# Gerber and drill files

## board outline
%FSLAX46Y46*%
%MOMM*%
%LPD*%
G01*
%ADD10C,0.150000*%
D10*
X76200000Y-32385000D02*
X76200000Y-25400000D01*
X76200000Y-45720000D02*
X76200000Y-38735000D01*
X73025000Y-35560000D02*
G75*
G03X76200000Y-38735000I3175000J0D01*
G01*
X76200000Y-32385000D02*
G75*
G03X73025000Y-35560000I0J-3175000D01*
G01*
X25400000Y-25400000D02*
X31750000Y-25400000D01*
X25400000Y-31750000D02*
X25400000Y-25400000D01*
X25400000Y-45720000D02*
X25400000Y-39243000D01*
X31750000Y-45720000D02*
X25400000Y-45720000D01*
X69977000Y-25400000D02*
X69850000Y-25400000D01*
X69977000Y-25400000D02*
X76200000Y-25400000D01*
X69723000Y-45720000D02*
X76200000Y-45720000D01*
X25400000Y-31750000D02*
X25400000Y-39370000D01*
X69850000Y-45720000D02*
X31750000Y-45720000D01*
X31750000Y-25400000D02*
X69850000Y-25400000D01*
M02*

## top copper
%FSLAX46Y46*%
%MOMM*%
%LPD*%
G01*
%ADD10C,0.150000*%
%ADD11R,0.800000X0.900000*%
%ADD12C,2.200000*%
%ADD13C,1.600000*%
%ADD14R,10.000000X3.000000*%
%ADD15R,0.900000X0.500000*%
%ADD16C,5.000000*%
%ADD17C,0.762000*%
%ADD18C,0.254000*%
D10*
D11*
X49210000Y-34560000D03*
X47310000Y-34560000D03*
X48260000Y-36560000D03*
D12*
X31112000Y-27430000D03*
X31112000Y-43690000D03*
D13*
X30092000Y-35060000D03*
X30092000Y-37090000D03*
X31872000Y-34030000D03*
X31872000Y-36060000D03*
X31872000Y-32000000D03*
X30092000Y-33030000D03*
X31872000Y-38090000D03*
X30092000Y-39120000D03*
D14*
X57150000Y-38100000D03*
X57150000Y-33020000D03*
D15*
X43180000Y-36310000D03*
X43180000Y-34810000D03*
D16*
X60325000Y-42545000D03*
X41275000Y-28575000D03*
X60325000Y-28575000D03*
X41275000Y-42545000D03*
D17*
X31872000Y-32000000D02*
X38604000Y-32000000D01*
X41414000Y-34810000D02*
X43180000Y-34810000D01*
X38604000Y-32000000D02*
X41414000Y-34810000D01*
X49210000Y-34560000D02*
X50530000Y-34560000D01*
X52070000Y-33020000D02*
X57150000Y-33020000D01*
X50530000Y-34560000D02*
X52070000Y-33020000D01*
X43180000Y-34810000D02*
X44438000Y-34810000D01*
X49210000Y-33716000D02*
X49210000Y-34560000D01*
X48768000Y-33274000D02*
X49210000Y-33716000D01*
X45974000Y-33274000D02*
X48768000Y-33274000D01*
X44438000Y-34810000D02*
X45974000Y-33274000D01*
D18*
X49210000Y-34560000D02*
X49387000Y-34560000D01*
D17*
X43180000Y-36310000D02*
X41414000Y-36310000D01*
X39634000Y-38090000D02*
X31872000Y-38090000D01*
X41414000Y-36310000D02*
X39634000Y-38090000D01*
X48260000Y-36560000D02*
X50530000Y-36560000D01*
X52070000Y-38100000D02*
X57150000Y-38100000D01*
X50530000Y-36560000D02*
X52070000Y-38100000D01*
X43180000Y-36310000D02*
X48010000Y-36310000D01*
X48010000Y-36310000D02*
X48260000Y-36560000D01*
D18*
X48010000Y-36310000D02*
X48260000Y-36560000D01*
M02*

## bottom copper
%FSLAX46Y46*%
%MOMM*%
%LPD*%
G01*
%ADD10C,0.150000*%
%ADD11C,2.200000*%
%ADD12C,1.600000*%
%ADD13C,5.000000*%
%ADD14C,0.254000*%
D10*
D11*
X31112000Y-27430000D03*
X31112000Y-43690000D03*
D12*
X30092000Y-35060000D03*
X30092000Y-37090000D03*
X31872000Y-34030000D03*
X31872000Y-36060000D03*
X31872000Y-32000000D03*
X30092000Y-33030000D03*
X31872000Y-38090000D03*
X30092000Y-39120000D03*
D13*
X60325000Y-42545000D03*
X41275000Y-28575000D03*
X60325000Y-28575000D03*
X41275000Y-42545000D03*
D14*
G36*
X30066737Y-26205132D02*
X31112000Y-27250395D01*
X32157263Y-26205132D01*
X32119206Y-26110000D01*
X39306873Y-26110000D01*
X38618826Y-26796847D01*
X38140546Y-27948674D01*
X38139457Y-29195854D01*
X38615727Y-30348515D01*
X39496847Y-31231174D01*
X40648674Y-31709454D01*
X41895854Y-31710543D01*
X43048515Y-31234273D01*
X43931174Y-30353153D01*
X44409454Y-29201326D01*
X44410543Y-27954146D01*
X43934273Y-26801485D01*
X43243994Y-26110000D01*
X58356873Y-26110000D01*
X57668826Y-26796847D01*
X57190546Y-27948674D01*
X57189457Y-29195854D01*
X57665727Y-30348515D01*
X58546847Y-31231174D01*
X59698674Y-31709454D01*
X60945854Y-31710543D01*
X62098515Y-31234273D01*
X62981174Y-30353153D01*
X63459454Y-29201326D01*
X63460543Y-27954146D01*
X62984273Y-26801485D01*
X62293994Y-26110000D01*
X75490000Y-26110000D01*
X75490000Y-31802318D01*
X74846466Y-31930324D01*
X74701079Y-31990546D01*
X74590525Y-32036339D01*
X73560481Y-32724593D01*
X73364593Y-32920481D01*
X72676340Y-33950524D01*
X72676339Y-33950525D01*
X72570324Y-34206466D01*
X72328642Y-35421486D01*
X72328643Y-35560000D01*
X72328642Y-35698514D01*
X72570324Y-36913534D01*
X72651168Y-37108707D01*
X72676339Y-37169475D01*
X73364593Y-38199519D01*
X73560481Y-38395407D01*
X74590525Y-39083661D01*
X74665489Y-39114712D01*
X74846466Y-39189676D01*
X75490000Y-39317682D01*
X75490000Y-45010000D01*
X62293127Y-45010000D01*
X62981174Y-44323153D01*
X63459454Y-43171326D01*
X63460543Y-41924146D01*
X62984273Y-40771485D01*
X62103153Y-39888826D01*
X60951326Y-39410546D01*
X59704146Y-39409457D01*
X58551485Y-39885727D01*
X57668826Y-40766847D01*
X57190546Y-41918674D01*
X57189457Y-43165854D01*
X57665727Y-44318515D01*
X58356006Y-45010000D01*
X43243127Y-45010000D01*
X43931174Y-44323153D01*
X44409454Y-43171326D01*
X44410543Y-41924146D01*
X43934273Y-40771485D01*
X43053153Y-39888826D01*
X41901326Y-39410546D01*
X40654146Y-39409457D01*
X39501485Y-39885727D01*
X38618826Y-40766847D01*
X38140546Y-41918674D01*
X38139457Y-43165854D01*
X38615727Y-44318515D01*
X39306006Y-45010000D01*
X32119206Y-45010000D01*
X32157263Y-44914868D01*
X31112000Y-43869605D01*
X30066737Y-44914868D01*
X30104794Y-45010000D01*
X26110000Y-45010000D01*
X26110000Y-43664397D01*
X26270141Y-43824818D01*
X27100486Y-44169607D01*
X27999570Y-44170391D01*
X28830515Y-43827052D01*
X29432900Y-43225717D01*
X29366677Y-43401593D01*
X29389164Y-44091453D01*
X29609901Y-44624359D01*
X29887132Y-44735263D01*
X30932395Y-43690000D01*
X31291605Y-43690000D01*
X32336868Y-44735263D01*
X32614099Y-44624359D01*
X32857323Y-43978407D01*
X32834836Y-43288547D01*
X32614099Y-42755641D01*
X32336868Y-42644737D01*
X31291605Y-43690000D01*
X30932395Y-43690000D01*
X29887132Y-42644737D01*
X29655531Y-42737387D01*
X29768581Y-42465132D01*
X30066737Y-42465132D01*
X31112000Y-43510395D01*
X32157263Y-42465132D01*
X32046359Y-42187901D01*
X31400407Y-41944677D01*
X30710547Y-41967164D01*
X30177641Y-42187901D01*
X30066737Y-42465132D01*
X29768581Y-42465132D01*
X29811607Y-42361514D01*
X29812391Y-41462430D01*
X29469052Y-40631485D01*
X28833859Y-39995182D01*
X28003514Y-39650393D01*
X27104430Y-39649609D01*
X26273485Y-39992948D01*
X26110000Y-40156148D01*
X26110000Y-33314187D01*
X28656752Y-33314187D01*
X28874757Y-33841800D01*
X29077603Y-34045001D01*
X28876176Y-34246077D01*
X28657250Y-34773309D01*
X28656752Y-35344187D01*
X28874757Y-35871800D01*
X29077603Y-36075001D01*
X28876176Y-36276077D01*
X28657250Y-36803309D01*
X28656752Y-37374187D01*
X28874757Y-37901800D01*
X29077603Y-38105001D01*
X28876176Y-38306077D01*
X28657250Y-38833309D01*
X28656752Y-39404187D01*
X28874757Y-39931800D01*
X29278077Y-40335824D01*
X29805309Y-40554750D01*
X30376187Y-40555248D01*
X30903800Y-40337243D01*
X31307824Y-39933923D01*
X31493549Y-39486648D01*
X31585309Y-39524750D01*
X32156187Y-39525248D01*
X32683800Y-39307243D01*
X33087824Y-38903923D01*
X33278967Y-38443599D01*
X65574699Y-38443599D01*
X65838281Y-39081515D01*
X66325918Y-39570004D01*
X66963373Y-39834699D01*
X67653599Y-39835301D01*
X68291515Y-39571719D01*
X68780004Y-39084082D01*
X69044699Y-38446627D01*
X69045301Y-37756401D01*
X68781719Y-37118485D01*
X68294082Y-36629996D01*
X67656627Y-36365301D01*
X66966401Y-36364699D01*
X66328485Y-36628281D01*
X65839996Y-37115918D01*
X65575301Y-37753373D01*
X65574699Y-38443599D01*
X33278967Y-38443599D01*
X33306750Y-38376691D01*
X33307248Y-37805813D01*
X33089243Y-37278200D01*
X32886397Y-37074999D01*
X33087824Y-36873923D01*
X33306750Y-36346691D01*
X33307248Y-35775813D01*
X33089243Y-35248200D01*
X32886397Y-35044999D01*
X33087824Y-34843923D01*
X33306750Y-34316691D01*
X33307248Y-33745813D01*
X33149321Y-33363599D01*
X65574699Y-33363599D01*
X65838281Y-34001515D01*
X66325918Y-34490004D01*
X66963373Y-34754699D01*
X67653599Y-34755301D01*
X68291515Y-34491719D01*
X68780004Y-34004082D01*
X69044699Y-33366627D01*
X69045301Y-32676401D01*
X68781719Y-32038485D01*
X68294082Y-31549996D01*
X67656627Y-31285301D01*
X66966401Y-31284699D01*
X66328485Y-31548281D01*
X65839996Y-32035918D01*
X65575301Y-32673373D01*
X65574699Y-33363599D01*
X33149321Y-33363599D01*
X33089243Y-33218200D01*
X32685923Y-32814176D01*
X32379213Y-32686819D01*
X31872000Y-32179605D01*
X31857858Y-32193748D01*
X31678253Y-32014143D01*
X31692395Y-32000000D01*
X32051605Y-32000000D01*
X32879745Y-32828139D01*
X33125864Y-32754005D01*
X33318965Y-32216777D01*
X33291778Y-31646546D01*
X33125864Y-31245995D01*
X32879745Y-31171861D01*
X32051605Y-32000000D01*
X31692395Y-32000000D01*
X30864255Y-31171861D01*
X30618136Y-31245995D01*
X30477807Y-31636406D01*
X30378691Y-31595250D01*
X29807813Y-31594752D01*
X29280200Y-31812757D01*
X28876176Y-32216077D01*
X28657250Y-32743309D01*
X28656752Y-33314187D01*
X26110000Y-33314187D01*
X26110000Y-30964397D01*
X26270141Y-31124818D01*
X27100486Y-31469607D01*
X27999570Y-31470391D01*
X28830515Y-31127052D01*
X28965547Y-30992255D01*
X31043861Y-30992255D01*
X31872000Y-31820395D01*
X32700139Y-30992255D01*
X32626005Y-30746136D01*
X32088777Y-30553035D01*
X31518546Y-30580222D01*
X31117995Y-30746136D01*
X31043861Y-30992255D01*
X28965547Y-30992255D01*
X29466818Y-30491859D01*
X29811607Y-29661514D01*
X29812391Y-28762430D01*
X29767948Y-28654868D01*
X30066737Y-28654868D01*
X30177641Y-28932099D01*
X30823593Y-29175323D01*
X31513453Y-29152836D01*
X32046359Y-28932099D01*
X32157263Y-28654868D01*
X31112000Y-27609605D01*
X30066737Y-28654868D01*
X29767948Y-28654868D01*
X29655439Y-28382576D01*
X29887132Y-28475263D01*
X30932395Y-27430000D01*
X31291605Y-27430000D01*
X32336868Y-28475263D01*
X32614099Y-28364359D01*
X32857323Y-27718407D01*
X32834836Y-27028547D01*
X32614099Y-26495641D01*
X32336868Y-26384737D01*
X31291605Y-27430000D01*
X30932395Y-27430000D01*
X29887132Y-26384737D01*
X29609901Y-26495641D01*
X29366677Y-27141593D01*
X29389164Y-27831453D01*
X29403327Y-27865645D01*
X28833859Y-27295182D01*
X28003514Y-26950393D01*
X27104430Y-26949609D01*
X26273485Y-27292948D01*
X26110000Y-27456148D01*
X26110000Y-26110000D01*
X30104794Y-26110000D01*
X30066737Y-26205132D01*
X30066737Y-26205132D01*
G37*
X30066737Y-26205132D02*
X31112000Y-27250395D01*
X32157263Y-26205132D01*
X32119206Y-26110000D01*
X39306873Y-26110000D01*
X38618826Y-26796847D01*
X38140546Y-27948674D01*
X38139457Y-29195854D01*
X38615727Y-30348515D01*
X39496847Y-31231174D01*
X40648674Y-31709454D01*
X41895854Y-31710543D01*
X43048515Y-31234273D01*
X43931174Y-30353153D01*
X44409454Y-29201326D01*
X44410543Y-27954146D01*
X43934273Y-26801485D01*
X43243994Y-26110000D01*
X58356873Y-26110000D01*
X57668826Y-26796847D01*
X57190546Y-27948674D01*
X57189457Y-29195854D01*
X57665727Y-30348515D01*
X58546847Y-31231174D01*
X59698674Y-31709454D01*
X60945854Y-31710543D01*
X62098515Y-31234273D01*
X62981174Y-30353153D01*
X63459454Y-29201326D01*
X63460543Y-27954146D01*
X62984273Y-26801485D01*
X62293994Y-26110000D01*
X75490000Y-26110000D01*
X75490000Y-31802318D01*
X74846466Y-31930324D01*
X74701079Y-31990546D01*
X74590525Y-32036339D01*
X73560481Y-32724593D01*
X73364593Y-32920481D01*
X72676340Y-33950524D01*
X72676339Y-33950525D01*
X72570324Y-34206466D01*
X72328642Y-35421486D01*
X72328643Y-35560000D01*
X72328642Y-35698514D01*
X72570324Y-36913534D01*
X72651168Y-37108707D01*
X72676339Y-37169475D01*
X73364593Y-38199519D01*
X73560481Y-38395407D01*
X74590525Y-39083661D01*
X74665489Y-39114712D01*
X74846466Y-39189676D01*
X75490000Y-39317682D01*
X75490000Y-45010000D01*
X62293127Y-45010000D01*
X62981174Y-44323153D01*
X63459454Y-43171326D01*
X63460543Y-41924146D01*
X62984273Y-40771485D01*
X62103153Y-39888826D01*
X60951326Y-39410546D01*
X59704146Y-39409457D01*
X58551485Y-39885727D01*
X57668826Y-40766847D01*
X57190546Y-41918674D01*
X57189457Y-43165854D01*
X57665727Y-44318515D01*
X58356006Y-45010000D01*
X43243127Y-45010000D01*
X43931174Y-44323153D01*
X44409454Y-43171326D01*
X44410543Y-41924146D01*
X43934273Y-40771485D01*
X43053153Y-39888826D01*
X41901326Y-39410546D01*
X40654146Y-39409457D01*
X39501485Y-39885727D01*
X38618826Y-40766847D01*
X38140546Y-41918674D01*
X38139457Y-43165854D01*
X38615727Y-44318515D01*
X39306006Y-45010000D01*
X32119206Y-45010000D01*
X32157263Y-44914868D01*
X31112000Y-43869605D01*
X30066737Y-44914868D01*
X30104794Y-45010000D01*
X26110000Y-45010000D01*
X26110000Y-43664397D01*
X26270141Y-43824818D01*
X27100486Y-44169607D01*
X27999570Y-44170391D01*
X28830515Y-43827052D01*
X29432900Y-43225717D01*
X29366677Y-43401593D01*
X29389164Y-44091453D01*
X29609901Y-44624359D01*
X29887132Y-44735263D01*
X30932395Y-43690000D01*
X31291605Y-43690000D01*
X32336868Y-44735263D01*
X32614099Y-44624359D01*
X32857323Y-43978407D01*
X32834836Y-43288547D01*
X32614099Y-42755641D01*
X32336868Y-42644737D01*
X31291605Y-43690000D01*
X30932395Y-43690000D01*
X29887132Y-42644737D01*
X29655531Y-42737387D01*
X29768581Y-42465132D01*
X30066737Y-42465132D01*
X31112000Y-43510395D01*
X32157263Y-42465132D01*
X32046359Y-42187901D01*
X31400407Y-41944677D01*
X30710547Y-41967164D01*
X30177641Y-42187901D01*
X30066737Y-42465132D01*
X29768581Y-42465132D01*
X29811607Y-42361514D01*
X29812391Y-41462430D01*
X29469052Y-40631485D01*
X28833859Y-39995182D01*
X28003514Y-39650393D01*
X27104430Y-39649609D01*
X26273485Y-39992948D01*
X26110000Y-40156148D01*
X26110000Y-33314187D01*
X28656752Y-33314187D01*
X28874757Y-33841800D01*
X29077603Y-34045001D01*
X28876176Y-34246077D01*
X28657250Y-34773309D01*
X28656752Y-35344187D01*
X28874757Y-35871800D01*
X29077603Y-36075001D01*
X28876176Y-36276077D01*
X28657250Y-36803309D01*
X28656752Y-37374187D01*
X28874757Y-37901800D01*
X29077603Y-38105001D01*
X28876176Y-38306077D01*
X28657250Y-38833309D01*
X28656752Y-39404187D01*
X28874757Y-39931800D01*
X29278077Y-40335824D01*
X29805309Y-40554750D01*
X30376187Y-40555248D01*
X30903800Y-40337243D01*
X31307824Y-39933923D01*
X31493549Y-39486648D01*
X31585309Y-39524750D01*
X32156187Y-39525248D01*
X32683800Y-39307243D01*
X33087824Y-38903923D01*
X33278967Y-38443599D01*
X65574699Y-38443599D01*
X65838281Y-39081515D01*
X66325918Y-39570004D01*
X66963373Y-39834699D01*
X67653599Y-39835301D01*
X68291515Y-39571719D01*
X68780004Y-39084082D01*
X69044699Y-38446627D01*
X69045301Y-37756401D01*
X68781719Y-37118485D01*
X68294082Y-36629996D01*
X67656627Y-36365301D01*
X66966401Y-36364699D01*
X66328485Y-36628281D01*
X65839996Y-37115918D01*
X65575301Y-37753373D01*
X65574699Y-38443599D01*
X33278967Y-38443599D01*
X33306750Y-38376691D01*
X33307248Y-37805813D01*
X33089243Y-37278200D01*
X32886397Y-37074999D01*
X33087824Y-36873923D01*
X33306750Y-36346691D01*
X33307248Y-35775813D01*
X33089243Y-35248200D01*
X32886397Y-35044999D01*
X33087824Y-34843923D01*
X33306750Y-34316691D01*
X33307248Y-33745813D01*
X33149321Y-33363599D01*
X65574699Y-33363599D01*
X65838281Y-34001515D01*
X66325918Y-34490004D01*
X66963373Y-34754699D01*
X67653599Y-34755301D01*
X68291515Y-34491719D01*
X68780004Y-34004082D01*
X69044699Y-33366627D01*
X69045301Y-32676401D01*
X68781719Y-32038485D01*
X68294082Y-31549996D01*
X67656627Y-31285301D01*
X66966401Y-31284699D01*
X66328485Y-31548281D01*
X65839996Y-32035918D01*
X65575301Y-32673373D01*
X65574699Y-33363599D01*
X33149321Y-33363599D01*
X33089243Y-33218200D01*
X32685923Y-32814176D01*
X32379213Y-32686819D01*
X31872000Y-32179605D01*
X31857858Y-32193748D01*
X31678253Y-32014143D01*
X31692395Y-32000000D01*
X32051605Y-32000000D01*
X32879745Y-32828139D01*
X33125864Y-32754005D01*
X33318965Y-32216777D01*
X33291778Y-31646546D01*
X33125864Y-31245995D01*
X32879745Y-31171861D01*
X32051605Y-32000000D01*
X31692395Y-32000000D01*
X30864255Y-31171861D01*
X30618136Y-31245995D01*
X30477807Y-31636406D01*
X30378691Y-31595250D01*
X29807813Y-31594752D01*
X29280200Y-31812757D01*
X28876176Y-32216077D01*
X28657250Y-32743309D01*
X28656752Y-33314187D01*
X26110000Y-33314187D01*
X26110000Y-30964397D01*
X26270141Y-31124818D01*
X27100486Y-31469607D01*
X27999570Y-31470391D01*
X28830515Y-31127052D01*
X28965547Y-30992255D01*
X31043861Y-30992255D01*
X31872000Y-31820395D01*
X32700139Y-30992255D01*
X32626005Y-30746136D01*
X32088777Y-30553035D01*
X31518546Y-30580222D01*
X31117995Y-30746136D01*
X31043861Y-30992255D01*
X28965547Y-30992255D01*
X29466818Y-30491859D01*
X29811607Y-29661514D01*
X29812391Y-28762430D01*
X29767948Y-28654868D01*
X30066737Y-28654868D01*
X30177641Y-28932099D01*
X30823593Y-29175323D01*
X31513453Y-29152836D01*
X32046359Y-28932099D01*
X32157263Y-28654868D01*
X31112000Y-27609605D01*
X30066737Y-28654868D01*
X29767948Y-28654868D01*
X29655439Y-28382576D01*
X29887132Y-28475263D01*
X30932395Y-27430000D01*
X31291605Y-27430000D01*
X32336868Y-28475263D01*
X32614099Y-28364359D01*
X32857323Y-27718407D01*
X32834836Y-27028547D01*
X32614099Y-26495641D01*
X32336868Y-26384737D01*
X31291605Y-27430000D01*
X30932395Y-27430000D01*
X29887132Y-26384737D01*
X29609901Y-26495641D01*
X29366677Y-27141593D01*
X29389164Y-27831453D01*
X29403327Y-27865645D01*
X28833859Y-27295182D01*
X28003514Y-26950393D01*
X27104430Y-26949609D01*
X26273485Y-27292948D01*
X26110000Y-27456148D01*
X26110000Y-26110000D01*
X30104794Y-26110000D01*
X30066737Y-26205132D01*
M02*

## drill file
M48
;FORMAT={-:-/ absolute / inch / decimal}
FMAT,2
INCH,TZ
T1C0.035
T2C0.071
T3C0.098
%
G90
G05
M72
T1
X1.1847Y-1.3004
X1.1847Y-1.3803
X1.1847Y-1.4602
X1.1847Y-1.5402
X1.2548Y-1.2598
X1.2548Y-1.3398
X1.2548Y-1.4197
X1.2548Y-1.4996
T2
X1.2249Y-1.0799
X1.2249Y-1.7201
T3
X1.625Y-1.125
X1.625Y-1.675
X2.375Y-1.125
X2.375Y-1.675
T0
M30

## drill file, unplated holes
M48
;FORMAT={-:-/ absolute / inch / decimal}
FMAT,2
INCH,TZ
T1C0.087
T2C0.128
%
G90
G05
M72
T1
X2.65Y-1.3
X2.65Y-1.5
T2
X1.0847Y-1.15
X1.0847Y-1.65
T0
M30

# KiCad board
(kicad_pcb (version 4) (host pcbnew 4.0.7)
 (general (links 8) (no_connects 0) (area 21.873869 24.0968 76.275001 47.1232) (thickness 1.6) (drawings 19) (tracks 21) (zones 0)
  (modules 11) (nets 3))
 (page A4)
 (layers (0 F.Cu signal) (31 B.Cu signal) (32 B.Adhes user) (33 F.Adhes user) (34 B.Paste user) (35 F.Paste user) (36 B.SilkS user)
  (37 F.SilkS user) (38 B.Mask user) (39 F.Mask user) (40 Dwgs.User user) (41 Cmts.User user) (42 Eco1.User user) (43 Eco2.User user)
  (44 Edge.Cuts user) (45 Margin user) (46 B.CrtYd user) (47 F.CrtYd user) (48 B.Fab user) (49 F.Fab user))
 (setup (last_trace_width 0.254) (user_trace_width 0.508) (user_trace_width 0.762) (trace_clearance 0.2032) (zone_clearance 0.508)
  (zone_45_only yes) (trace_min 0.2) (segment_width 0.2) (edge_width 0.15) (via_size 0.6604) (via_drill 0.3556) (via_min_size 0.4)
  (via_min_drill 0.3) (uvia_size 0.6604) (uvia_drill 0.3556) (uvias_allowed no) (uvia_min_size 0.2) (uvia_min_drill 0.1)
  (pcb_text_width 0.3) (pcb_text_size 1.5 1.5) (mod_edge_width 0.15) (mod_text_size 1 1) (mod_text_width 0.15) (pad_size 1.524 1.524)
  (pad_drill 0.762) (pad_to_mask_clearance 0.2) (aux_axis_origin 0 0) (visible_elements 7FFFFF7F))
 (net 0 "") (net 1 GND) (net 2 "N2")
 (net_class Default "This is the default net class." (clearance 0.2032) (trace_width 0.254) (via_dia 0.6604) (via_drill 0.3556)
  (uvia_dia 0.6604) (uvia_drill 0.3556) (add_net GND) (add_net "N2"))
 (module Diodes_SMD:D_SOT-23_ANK (layer F.Cu) (at 48.26 35.56 270)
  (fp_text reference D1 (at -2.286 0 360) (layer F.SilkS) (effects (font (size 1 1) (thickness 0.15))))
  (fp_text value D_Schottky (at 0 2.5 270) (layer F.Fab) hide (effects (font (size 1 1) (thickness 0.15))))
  (pad 2 smd rect (at -1 -0.95 270) (size 0.9 0.8) (layers F.Cu F.Paste F.Mask) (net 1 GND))
  (pad "" smd rect (at -1 0.95 270) (size 0.9 0.8) (layers F.Cu F.Paste F.Mask))
  (pad 1 smd rect (at 1 0 270) (size 0.9 0.8) (layers F.Cu F.Paste F.Mask) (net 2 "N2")))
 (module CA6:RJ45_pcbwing (layer F.Cu) (at 29.972 35.56 270)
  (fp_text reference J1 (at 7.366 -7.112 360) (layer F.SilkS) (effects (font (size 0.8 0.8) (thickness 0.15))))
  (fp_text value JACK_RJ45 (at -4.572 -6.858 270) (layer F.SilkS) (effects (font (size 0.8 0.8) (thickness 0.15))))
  (pad 8 thru_hole circle (at -8.13 -1.14 270) (size 2.2 2.2) (drill 1.8) (layers *.Cu *.Mask F.SilkS) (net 1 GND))
  (pad 8 thru_hole circle (at 8.13 -1.14 270) (size 2.2 2.2) (drill 1.8) (layers *.Cu *.Mask F.SilkS) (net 1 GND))
  (pad "" np_thru_hole circle (at -6.35 2.42 270) (size 3.25 3.25) (drill 3.25) (layers *.Cu *.Mask F.SilkS))
  (pad "" np_thru_hole circle (at 6.35 2.42 270) (size 3.25 3.25) (drill 3.25) (layers *.Cu *.Mask F.SilkS))
  (pad 5 thru_hole circle (at -0.5 -0.12 270) (size 1.6 1.6) (drill 0.89) (layers *.Cu *.Mask F.SilkS))
  (pad 3 thru_hole circle (at 1.53 -0.12 270) (size 1.6 1.6) (drill 0.89) (layers *.Cu *.Mask F.SilkS))
  (pad 6 thru_hole circle (at -1.53 -1.9 270) (size 1.6 1.6) (drill 0.89) (layers *.Cu *.Mask F.SilkS))
  (pad 4 thru_hole circle (at 0.5 -1.9 270) (size 1.6 1.6) (drill 0.89) (layers *.Cu *.Mask F.SilkS))
  (pad 8 thru_hole circle (at -3.56 -1.9 270) (size 1.6 1.6) (drill 0.89) (layers *.Cu *.Mask F.SilkS) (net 1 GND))
  (pad 7 thru_hole circle (at -2.53 -0.12 270) (size 1.6 1.6) (drill 0.89) (layers *.Cu *.Mask F.SilkS))
  (pad 2 thru_hole circle (at 2.53 -1.9 270) (size 1.6 1.6) (drill 0.89) (layers *.Cu *.Mask F.SilkS) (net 2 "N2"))
  (pad 1 thru_hole circle (at 3.56 -0.12 270) (size 1.6 1.6) (drill 0.89) (layers *.Cu *.Mask F.SilkS)))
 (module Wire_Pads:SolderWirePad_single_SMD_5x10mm (layer F.Cu) (at 57.15 38.1 90)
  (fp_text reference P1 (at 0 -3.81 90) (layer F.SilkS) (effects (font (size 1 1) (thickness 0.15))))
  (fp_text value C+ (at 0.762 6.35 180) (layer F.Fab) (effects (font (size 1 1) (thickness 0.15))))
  (pad 1 smd rect (at 0 0 90) (size 3 10) (layers F.Cu F.Paste F.Mask) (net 2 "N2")))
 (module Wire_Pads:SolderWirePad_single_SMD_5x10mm (layer F.Cu) (at 57.15 33.02 90)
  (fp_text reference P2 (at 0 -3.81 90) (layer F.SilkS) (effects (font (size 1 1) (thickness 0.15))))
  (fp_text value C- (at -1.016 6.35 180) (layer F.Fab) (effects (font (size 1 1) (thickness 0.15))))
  (pad 1 smd rect (at 0 0 90) (size 3 10) (layers F.Cu F.Paste F.Mask) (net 1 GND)))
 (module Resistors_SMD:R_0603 (layer F.Cu) (at 43.18 35.56 90)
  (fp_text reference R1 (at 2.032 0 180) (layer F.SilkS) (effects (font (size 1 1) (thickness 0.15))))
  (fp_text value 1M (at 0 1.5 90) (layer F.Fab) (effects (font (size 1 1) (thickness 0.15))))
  (pad 1 smd rect (at -0.75 0 90) (size 0.5 0.9) (layers F.Cu F.Paste F.Mask) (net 2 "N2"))
  (pad 2 smd rect (at 0.75 0 90) (size 0.5 0.9) (layers F.Cu F.Paste F.Mask) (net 1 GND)))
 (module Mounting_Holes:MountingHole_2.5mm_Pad (layer F.Cu) (at 60.325 42.545)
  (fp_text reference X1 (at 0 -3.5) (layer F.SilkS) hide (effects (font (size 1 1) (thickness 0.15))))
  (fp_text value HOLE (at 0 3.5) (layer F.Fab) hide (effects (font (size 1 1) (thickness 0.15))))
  (pad 1 thru_hole circle (at 0 0) (size 5 5) (drill 2.5) (layers *.Cu *.Mask)))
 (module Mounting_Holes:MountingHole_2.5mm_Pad (layer F.Cu) (at 41.275 28.575)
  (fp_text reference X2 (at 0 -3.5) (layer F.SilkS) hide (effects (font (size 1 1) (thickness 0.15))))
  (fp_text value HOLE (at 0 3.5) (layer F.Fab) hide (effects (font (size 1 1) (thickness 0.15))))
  (pad 1 thru_hole circle (at 0 0) (size 5 5) (drill 2.5) (layers *.Cu *.Mask)))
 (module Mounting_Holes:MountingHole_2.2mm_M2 (layer F.Cu) (at 67.31 38.1)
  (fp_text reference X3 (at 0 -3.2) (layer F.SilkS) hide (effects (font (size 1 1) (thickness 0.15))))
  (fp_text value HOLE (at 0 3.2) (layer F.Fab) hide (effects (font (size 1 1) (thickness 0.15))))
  (pad 1 np_thru_hole circle (at 0 0) (size 2.2 2.2) (drill 2.2) (layers *.Cu *.Mask)))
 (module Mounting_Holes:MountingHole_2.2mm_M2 (layer F.Cu) (at 67.31 33.02)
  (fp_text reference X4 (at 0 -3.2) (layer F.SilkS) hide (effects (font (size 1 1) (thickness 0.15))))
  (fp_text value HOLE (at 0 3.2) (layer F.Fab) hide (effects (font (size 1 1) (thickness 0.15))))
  (pad 1 np_thru_hole circle (at 0 0) (size 2.2 2.2) (drill 2.2) (layers *.Cu *.Mask)))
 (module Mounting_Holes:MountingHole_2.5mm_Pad (layer F.Cu) (at 60.325 28.575)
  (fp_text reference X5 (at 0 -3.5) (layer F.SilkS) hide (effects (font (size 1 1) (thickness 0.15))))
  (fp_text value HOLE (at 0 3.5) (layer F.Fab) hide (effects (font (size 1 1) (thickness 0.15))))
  (pad 1 thru_hole circle (at 0 0) (size 5 5) (drill 2.5) (layers *.Cu *.Mask)))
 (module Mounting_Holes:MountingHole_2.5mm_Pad (layer F.Cu) (at 41.275 42.545)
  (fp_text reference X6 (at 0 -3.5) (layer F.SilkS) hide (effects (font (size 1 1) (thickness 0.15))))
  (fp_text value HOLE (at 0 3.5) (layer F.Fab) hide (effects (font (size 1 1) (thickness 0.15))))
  (pad 1 thru_hole circle (at 0 0) (size 5 5) (drill 2.5) (layers *.Cu *.Mask)))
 (gr_line (start 76.2 32.385) (end 76.2 25.4) (angle 90) (layer Edge.Cuts) (width 0.15))
 (gr_line (start 76.2 45.72) (end 76.2 38.735) (angle 90) (layer Edge.Cuts) (width 0.15))
 (gr_arc (start 76.2 35.56) (end 76.2 38.735) (angle 90) (layer Edge.Cuts) (width 0.15))
 (gr_arc (start 76.2 35.56) (end 73.025 35.56) (angle 90) (layer Edge.Cuts) (width 0.15))
 (gr_line (start 25.4 25.4) (end 31.75 25.4) (angle 90) (layer Edge.Cuts) (width 0.15))
 (gr_line (start 25.4 31.75) (end 25.4 25.4) (angle 90) (layer Edge.Cuts) (width 0.15))
 (gr_line (start 25.4 45.72) (end 25.4 39.243) (angle 90) (layer Edge.Cuts) (width 0.15))
 (gr_line (start 31.75 45.72) (end 25.4 45.72) (angle 90) (layer Edge.Cuts) (width 0.15))
 (gr_line (start 69.977 25.4) (end 69.85 25.4) (angle 90) (layer Edge.Cuts) (width 0.15))
 (gr_line (start 69.977 25.4) (end 76.2 25.4) (angle 90) (layer Edge.Cuts) (width 0.15))
 (gr_line (start 69.723 45.72) (end 76.2 45.72) (angle 90) (layer Edge.Cuts) (width 0.15))
 (gr_line (start 25.4 31.75) (end 25.4 39.37) (angle 90) (layer Edge.Cuts) (width 0.15))
 (gr_line (start 69.85 45.72) (end 31.75 45.72) (angle 90) (layer Edge.Cuts) (width 0.15))
 (gr_line (start 31.75 25.4) (end 69.85 25.4) (angle 90) (layer Edge.Cuts) (width 0.15))
 (segment (start 31.872 32) (end 38.604 32) (width 0.762) (layer F.Cu) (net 1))
 (segment (start 41.414 34.81) (end 43.18 34.81) (width 0.762) (layer F.Cu) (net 1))
 (segment (start 38.604 32) (end 41.414 34.81) (width 0.762) (layer F.Cu) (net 1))
 (segment (start 49.21 34.56) (end 50.53 34.56) (width 0.762) (layer F.Cu) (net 1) (status 10))
 (segment (start 52.07 33.02) (end 57.15 33.02) (width 0.762) (layer F.Cu) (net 1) (status 20))
 (segment (start 50.53 34.56) (end 52.07 33.02) (width 0.762) (layer F.Cu) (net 1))
 (segment (start 43.18 34.81) (end 44.438 34.81) (width 0.762) (layer F.Cu) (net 1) (status 10))
 (segment (start 49.21 33.716) (end 49.21 34.56) (width 0.762) (layer F.Cu) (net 1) (status 20))
 (segment (start 48.768 33.274) (end 49.21 33.716) (width 0.762) (layer F.Cu) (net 1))
 (segment (start 45.974 33.274) (end 48.768 33.274) (width 0.762) (layer F.Cu) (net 1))
 (segment (start 44.438 34.81) (end 45.974 33.274) (width 0.762) (layer F.Cu) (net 1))
 (segment (start 49.21 34.56) (end 49.387 34.56) (width 0.254) (layer F.Cu) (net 1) (status 30))
 (segment (start 43.18 36.31) (end 41.414 36.31) (width 0.762) (layer F.Cu) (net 2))
 (segment (start 39.634 38.09) (end 31.872 38.09) (width 0.762) (layer F.Cu) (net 2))
 (segment (start 41.414 36.31) (end 39.634 38.09) (width 0.762) (layer F.Cu) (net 2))
 (segment (start 48.26 36.56) (end 50.53 36.56) (width 0.762) (layer F.Cu) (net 2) (status 10))
 (segment (start 52.07 38.1) (end 57.15 38.1) (width 0.762) (layer F.Cu) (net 2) (status 20))
 (segment (start 50.53 36.56) (end 52.07 38.1) (width 0.762) (layer F.Cu) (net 2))
 (segment (start 43.18 36.31) (end 48.01 36.31) (width 0.762) (layer F.Cu) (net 2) (status 30))
 (segment (start 48.01 36.31) (end 48.26 36.56) (width 0.762) (layer F.Cu) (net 2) (status 30))
 (segment (start 48.01 36.31) (end 48.26 36.56) (width 0.254) (layer F.Cu) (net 2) (status 30))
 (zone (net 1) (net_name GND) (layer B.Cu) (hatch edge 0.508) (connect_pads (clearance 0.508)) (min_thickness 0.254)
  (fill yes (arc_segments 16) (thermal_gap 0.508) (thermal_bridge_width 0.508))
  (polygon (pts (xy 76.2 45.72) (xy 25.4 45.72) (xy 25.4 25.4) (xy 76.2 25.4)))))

